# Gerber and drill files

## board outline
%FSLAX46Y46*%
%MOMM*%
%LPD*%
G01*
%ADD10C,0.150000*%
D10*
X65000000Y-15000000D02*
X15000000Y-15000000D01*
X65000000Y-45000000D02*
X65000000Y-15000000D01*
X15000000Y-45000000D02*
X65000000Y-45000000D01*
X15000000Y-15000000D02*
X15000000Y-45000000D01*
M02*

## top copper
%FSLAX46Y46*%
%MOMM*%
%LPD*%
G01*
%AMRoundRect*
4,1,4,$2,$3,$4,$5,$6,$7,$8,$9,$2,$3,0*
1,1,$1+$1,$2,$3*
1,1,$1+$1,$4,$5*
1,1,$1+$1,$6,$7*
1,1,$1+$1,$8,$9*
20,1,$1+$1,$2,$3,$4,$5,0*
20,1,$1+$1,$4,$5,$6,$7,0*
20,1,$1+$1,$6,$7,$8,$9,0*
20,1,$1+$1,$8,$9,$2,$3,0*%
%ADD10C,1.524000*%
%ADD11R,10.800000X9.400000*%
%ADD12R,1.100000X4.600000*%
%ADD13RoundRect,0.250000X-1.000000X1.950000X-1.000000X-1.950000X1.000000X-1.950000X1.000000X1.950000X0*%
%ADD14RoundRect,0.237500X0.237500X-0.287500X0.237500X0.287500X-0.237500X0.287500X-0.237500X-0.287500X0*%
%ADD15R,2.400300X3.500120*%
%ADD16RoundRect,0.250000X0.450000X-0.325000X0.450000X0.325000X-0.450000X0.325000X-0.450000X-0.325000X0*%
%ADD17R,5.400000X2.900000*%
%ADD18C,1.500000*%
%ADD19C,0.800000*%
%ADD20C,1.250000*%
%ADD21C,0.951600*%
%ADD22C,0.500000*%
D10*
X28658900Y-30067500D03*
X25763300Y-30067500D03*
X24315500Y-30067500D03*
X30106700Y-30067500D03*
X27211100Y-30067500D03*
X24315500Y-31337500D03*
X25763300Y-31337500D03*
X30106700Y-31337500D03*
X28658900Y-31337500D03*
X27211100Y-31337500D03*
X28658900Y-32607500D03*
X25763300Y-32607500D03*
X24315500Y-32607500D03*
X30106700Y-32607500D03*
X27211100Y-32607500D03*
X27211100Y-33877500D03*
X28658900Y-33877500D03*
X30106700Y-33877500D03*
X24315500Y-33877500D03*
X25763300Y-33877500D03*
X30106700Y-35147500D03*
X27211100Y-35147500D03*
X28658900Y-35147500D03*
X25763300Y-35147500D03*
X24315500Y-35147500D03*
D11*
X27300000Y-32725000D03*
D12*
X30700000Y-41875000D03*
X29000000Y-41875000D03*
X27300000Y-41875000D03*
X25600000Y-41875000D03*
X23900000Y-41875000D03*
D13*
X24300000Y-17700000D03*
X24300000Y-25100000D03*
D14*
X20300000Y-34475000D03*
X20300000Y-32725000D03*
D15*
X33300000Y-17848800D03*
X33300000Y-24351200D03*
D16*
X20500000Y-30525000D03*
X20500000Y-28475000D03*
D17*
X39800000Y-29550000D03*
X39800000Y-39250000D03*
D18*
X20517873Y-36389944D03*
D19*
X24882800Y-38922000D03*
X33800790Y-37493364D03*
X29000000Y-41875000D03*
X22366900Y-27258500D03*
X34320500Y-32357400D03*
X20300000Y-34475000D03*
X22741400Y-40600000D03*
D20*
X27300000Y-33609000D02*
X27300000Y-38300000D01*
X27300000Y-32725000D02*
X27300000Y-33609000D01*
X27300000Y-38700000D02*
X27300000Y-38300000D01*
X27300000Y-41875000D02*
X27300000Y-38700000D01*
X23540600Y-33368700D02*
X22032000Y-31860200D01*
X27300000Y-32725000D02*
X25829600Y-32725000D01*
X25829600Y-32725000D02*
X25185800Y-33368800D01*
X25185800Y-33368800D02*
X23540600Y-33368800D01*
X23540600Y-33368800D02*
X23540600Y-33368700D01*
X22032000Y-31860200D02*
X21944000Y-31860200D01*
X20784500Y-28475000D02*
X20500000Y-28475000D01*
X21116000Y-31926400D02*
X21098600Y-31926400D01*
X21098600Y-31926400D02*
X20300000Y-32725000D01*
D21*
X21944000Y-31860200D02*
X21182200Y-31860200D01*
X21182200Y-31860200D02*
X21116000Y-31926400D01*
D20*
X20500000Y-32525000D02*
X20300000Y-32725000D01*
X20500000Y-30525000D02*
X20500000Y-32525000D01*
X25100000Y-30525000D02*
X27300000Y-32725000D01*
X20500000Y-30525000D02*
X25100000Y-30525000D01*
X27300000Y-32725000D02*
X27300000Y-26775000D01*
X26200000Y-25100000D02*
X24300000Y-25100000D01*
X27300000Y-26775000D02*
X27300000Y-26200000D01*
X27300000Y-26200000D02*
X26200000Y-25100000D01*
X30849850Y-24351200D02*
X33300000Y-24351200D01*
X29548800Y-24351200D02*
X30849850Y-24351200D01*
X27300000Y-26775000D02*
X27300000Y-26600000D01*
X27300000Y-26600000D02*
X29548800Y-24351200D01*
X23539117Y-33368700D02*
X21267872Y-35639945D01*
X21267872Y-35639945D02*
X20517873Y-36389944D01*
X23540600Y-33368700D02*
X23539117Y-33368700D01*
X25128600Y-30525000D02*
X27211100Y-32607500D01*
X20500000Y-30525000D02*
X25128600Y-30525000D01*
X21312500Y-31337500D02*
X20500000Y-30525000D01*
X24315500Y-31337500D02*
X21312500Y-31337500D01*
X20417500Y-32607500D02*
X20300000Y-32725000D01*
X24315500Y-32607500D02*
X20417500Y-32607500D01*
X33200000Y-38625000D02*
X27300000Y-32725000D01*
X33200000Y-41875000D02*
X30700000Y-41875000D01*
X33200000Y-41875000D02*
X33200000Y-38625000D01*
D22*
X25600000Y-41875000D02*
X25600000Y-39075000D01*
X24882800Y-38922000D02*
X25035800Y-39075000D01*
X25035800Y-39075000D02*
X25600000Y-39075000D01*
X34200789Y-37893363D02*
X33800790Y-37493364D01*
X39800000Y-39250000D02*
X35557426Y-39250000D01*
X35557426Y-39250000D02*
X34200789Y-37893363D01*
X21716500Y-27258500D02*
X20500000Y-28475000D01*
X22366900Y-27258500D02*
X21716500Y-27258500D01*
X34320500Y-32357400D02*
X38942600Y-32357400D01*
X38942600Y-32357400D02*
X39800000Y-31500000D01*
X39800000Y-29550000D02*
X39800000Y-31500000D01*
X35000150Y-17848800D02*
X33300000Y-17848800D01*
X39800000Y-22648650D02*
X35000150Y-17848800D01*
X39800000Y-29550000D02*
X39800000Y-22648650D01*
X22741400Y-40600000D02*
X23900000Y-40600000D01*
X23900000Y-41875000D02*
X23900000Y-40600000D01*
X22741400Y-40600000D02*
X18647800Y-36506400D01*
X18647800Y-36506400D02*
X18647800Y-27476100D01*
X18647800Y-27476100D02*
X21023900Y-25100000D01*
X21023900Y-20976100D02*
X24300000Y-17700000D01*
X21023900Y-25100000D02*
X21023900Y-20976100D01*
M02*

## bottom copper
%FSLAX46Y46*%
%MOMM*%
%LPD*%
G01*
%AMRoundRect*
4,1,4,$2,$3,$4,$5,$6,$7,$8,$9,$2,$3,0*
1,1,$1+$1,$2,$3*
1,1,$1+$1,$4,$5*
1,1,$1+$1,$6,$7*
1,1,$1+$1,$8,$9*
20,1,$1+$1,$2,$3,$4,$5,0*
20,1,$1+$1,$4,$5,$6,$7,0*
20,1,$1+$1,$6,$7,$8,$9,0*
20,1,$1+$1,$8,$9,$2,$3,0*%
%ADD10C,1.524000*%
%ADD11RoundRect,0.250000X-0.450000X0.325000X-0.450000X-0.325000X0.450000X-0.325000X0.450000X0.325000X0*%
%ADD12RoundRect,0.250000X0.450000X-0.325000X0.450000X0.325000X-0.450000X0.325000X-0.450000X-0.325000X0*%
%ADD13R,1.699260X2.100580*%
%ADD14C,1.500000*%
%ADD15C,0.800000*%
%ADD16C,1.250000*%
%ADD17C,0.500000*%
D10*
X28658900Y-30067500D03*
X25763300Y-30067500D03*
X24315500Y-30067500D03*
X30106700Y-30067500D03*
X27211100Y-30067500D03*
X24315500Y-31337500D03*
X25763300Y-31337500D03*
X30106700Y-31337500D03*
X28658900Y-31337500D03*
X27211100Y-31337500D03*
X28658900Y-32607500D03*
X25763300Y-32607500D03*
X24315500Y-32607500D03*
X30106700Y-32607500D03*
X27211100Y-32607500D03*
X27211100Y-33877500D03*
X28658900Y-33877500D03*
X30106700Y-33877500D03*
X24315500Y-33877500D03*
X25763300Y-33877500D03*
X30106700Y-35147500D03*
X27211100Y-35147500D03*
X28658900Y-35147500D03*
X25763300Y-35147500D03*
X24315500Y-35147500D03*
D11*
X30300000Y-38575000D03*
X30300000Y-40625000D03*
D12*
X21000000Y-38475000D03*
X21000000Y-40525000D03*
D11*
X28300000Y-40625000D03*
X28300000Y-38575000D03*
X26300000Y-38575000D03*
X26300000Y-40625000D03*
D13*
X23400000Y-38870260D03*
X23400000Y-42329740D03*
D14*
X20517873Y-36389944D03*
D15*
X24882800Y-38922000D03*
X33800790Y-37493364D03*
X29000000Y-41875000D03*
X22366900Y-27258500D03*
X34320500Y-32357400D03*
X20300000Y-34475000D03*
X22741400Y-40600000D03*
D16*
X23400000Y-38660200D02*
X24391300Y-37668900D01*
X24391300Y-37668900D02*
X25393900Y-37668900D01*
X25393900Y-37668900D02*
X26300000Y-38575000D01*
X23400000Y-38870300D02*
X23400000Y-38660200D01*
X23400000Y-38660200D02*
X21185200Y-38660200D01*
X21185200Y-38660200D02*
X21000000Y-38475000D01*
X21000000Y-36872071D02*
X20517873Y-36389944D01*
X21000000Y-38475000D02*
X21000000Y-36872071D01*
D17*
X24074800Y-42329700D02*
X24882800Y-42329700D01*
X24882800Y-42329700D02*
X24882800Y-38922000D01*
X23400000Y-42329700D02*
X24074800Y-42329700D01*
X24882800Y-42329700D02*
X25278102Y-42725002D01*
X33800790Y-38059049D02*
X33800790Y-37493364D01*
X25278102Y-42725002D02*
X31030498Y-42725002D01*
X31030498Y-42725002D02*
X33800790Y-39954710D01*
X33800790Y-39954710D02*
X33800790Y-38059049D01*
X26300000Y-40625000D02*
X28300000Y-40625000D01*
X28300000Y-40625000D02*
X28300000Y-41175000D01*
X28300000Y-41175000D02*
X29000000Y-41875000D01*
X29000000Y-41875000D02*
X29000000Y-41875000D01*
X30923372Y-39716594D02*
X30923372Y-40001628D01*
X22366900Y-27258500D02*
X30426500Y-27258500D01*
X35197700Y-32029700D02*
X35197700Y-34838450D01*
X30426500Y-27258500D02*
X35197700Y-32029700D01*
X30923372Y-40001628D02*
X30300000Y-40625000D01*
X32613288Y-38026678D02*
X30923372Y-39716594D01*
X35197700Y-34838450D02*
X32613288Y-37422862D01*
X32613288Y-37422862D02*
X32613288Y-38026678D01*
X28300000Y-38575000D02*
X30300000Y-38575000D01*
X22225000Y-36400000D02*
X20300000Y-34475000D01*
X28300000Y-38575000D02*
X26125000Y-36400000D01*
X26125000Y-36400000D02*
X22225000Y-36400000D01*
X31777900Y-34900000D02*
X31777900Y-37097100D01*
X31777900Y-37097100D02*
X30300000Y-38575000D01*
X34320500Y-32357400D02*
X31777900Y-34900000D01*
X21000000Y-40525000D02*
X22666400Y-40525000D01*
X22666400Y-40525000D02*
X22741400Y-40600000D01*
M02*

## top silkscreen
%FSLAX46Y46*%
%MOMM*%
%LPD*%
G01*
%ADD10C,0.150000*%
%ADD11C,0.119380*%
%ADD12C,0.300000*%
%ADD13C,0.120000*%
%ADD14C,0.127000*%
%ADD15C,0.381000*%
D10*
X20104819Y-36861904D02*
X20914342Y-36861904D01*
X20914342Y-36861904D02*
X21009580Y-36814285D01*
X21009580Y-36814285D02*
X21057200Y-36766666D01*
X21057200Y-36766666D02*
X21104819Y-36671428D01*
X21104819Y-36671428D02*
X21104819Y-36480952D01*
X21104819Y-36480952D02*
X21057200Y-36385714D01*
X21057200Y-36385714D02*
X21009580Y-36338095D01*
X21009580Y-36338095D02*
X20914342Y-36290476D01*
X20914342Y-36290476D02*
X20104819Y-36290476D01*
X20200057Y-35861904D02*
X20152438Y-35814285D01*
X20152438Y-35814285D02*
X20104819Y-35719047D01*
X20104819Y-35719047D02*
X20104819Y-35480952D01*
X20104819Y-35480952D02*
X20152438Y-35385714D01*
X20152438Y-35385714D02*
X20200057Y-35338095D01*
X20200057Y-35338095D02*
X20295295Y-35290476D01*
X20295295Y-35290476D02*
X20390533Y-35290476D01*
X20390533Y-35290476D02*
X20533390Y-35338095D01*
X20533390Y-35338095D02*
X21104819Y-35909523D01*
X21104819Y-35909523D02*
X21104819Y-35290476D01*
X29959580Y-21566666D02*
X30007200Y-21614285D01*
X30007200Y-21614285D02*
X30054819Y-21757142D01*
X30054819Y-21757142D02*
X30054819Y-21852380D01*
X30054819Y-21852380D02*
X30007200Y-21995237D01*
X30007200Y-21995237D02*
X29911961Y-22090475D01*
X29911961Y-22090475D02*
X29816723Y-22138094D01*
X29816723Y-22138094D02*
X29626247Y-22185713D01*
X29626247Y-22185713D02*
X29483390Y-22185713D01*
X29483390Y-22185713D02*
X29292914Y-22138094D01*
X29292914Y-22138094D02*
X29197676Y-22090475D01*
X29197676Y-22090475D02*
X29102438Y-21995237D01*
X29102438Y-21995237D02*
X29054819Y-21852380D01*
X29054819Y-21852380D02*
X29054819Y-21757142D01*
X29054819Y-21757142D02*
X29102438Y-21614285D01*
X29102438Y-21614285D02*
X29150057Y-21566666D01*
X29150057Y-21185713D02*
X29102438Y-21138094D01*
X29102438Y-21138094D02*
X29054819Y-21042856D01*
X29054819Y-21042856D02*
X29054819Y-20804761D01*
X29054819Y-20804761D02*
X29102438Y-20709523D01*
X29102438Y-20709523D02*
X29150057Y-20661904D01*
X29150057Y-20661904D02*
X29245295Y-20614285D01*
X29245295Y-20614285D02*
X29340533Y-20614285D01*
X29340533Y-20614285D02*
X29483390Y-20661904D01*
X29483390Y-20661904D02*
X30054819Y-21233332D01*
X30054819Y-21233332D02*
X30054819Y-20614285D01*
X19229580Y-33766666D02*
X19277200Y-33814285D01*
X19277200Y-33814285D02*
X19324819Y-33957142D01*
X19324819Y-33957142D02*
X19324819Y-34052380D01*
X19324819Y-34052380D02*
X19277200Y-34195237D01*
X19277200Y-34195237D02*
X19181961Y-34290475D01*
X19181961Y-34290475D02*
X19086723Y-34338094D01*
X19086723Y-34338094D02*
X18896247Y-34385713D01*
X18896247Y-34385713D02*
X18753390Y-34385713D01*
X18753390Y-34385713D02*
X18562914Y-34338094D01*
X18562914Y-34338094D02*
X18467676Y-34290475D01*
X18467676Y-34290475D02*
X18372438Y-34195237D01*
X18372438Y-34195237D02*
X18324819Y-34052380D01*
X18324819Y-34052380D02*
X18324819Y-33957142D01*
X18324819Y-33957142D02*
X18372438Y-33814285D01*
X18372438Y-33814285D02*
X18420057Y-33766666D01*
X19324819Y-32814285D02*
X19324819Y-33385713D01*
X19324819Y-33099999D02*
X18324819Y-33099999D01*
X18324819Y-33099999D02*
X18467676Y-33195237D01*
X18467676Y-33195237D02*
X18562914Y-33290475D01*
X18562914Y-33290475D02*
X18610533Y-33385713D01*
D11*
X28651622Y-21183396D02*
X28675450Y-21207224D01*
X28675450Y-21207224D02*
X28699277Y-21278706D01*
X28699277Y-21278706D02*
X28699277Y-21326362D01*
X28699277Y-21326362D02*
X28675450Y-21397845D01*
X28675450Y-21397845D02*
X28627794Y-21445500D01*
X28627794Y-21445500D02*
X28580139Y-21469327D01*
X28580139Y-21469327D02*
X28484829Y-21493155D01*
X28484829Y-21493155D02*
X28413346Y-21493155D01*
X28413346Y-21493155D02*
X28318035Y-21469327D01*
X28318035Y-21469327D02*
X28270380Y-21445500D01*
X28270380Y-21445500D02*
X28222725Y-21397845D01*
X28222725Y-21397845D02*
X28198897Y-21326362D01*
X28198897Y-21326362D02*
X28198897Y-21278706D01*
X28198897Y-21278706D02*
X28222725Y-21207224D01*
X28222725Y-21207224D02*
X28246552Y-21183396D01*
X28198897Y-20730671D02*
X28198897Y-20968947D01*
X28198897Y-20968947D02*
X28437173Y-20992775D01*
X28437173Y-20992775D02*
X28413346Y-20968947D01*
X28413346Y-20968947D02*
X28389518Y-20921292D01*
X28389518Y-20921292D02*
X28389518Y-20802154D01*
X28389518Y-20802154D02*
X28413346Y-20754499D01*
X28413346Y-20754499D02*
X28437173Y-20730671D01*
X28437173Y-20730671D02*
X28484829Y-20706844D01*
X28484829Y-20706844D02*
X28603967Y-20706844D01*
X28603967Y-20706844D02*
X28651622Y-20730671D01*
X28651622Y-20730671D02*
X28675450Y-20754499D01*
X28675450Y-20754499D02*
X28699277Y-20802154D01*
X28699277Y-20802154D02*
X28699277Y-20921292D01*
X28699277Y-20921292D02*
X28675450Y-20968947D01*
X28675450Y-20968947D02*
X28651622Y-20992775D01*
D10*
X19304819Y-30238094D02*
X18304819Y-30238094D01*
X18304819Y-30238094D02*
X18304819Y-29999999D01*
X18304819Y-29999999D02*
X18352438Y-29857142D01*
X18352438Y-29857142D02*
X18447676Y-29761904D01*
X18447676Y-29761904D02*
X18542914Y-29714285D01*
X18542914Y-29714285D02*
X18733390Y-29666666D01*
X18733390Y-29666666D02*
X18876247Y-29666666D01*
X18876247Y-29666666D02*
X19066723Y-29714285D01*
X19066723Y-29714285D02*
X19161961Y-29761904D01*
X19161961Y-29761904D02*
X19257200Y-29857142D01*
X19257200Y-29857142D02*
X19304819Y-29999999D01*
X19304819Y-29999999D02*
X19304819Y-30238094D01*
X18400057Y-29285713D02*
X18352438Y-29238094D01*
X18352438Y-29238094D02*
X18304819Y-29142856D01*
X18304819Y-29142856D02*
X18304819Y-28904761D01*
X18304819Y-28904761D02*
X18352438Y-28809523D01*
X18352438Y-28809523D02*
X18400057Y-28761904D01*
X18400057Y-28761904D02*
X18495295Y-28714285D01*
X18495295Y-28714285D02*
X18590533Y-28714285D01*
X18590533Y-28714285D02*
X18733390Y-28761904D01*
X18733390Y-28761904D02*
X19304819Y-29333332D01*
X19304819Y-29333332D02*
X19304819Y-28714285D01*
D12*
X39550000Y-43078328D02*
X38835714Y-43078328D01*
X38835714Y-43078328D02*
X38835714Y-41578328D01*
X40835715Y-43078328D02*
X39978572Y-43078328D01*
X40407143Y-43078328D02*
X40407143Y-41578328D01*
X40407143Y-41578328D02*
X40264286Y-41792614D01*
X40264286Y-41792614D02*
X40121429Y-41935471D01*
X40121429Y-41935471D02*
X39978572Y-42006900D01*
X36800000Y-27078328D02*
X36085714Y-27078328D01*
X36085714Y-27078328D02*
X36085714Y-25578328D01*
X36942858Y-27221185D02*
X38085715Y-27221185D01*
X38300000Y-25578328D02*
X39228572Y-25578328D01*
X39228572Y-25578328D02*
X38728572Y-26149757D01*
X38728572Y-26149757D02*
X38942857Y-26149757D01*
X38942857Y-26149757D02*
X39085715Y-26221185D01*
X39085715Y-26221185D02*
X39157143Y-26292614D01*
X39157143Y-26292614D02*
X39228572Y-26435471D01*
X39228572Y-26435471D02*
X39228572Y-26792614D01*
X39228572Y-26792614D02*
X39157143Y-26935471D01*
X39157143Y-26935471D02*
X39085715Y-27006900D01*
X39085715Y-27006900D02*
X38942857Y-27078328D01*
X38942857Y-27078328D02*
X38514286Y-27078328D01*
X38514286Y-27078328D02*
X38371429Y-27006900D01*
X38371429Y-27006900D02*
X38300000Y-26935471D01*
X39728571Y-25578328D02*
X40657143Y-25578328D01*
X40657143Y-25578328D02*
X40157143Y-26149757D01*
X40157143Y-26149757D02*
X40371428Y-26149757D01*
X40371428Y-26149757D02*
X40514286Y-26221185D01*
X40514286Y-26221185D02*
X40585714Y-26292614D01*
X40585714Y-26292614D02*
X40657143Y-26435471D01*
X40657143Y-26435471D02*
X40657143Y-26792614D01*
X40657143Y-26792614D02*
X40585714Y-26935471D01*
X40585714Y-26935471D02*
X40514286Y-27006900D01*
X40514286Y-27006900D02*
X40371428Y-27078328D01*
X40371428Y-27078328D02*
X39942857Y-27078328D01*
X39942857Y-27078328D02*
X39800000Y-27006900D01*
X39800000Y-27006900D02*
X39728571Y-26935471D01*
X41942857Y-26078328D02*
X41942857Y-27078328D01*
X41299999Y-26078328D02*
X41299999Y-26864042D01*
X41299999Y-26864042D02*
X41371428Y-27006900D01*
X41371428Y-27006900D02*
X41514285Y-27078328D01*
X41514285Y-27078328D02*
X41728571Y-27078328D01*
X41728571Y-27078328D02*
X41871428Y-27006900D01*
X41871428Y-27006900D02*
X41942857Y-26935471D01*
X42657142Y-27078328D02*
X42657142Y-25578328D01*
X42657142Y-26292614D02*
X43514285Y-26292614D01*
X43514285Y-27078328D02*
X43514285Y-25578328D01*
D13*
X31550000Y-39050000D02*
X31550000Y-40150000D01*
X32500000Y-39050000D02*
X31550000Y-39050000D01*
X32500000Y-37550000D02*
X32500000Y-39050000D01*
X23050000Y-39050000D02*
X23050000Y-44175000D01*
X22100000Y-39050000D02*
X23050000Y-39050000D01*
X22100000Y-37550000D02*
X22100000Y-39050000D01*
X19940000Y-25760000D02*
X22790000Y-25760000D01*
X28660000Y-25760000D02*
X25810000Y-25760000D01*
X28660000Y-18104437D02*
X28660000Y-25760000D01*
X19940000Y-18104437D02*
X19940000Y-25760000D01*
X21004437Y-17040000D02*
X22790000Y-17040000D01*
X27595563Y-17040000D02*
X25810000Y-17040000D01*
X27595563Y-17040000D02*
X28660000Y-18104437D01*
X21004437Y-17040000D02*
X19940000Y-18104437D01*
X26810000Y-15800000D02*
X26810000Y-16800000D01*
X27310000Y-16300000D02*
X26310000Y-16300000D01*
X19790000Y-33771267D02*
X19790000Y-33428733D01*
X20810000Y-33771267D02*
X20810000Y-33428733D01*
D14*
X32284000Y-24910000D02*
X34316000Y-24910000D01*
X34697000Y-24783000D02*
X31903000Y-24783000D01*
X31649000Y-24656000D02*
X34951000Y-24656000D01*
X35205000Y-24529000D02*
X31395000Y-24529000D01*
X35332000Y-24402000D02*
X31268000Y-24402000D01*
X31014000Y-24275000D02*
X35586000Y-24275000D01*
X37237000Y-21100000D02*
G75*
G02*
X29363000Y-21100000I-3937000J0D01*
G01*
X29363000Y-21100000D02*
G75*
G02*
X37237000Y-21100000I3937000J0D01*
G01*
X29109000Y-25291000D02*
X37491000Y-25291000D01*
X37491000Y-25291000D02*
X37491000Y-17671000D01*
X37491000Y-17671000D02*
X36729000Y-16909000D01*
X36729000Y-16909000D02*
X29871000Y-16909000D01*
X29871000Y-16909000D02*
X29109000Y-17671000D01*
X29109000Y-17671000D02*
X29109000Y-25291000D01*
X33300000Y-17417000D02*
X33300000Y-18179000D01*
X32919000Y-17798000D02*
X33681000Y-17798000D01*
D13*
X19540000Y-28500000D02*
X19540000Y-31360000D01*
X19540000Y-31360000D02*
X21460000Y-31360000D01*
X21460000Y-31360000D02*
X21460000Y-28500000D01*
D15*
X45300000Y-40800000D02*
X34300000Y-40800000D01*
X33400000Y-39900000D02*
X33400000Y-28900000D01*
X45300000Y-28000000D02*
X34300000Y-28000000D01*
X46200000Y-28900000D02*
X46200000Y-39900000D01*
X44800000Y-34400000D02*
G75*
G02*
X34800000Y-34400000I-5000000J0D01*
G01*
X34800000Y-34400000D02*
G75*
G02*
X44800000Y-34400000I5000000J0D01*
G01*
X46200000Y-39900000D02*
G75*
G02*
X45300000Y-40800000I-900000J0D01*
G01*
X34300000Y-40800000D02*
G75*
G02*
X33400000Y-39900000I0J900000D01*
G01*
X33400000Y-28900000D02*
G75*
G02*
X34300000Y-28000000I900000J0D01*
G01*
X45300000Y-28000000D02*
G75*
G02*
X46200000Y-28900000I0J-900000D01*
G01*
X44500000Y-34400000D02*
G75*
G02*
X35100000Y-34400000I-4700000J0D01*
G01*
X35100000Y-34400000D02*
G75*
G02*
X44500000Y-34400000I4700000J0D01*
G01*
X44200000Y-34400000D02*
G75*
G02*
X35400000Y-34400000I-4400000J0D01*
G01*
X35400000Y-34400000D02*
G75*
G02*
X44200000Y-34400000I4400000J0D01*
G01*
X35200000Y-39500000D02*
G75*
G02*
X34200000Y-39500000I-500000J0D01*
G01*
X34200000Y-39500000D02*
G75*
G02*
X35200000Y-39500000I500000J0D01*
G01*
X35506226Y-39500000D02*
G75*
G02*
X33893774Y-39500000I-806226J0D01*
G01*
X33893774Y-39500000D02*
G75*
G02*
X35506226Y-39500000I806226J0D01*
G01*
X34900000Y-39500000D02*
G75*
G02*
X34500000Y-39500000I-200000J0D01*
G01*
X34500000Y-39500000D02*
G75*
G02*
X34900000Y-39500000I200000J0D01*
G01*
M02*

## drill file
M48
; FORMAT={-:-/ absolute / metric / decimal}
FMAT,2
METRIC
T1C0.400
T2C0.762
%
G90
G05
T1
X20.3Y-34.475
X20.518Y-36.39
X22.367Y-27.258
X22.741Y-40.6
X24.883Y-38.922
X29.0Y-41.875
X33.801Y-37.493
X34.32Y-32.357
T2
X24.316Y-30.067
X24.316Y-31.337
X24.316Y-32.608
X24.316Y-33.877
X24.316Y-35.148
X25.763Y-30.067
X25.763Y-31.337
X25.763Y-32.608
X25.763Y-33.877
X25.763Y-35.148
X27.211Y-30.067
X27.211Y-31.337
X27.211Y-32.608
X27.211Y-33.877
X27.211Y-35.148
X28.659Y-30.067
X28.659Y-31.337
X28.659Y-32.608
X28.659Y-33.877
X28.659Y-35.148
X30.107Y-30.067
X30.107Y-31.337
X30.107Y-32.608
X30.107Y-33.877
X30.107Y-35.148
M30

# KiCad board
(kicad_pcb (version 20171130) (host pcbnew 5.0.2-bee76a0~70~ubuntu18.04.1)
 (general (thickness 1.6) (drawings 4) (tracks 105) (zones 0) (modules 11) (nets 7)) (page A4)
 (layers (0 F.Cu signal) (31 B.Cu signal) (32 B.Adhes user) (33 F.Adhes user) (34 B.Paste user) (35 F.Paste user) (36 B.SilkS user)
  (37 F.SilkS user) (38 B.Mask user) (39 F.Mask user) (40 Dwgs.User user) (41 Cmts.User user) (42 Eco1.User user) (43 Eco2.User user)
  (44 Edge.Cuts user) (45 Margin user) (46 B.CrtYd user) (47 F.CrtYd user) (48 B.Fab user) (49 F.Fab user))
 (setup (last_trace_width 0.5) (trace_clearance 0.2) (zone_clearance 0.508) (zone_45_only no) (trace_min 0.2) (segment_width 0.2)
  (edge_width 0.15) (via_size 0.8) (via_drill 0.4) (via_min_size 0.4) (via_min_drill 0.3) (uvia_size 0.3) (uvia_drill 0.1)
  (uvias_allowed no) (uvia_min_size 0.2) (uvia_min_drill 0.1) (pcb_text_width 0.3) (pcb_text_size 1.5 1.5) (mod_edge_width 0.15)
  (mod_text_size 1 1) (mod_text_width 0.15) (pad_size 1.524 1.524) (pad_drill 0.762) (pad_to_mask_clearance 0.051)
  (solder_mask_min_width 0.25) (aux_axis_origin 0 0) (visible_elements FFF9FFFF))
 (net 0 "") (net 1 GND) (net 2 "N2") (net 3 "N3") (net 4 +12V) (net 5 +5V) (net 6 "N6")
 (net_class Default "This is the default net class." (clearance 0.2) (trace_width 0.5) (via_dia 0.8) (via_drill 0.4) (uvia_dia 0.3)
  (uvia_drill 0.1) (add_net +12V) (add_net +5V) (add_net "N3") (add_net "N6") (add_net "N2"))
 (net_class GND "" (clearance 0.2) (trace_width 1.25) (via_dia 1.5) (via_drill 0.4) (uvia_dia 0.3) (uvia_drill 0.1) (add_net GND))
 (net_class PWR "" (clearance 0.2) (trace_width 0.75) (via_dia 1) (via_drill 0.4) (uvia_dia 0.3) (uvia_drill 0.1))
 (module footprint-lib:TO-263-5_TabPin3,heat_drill (layer F.Cu) (at 27.3 36.1 90)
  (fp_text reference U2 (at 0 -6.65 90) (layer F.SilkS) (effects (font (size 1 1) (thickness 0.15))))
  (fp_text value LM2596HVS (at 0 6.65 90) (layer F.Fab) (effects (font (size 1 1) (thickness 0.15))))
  (fp_line (start -2.95 4.25) (end -4.05 4.25) (layer F.SilkS) (width 0.12))
  (fp_line (start -2.95 5.2) (end -2.95 4.25) (layer F.SilkS) (width 0.12))
  (fp_line (start -1.45 5.2) (end -2.95 5.2) (layer F.SilkS) (width 0.12))
  (fp_line (start -2.95 -4.25) (end -8.075 -4.25) (layer F.SilkS) (width 0.12))
  (fp_line (start -2.95 -5.2) (end -2.95 -4.25) (layer F.SilkS) (width 0.12))
  (fp_line (start -1.45 -5.2) (end -2.95 -5.2) (layer F.SilkS) (width 0.12))
  (pad 3 thru_hole circle (at 6.0325 1.3589 90) (size 1.524 1.524) (drill 0.762) (layers *.Cu *.Mask) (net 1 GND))
  (pad 3 thru_hole circle (at 6.0325 -1.5367 90) (size 1.524 1.524) (drill 0.762) (layers *.Cu *.Mask) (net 1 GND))
  (pad 3 thru_hole circle (at 6.0325 -2.9845 90) (size 1.524 1.524) (drill 0.762) (layers *.Cu *.Mask) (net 1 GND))
  (pad 3 thru_hole circle (at 6.0325 2.8067 90) (size 1.524 1.524) (drill 0.762) (layers *.Cu *.Mask) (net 1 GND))
  (pad 3 thru_hole circle (at 6.0325 -0.0889 90) (size 1.524 1.524) (drill 0.762) (layers *.Cu *.Mask) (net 1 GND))
  (pad 3 thru_hole circle (at 4.7625 -2.9845 90) (size 1.524 1.524) (drill 0.762) (layers *.Cu *.Mask) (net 1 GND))
  (pad 3 thru_hole circle (at 4.7625 -1.5367 90) (size 1.524 1.524) (drill 0.762) (layers *.Cu *.Mask) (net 1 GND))
  (pad 3 thru_hole circle (at 4.7625 2.8067 90) (size 1.524 1.524) (drill 0.762) (layers *.Cu *.Mask) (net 1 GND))
  (pad 3 thru_hole circle (at 4.7625 1.3589 90) (size 1.524 1.524) (drill 0.762) (layers *.Cu *.Mask) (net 1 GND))
  (pad 3 thru_hole circle (at 4.7625 -0.0889 90) (size 1.524 1.524) (drill 0.762) (layers *.Cu *.Mask) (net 1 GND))
  (pad 3 thru_hole circle (at 3.4925 1.3589 90) (size 1.524 1.524) (drill 0.762) (layers *.Cu *.Mask) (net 1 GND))
  (pad 3 thru_hole circle (at 3.4925 -1.5367 90) (size 1.524 1.524) (drill 0.762) (layers *.Cu *.Mask) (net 1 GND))
  (pad 3 thru_hole circle (at 3.4925 -2.9845 90) (size 1.524 1.524) (drill 0.762) (layers *.Cu *.Mask) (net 1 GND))
  (pad 3 thru_hole circle (at 3.4925 2.8067 90) (size 1.524 1.524) (drill 0.762) (layers *.Cu *.Mask) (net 1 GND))
  (pad 3 thru_hole circle (at 3.4925 -0.0889 90) (size 1.524 1.524) (drill 0.762) (layers *.Cu *.Mask) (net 1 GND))
  (pad 3 thru_hole circle (at 2.2225 -0.0889 90) (size 1.524 1.524) (drill 0.762) (layers *.Cu *.Mask) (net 1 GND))
  (pad 3 thru_hole circle (at 2.2225 1.3589 90) (size 1.524 1.524) (drill 0.762) (layers *.Cu *.Mask) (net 1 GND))
  (pad 3 thru_hole circle (at 2.2225 2.8067 90) (size 1.524 1.524) (drill 0.762) (layers *.Cu *.Mask) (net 1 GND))
  (pad 3 thru_hole circle (at 2.2225 -2.9845 90) (size 1.524 1.524) (drill 0.762) (layers *.Cu *.Mask) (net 1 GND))
  (pad 3 thru_hole circle (at 2.2225 -1.5367 90) (size 1.524 1.524) (drill 0.762) (layers *.Cu *.Mask) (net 1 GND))
  (pad 3 thru_hole circle (at 0.9525 2.8067 90) (size 1.524 1.524) (drill 0.762) (layers *.Cu *.Mask) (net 1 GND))
  (pad 3 thru_hole circle (at 0.9525 -0.0889 90) (size 1.524 1.524) (drill 0.762) (layers *.Cu *.Mask) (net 1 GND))
  (pad 3 thru_hole circle (at 0.9525 1.3589 90) (size 1.524 1.524) (drill 0.762) (layers *.Cu *.Mask) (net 1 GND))
  (pad 3 thru_hole circle (at 0.9525 -1.5367 90) (size 1.524 1.524) (drill 0.762) (layers *.Cu *.Mask) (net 1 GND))
  (pad 3 thru_hole circle (at 0.9525 -2.9845 90) (size 1.524 1.524) (drill 0.762) (layers *.Cu *.Mask) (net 1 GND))
  (pad "" smd rect (at 0.95 2.775 90) (size 4.55 5.25) (layers F.Paste))
  (pad "" smd rect (at 5.8 -2.775 90) (size 4.55 5.25) (layers F.Paste))
  (pad "" smd rect (at 0.95 -2.775 90) (size 4.55 5.25) (layers F.Paste))
  (pad "" smd rect (at 5.8 2.775 90) (size 4.55 5.25) (layers F.Paste))
  (pad 3 smd rect (at 3.375 0 90) (size 9.4 10.8) (layers F.Cu F.Mask) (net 1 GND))
  (pad 5 smd rect (at -5.775 3.4 90) (size 4.6 1.1) (layers F.Cu F.Paste F.Mask) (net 1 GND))
  (pad 4 smd rect (at -5.775 1.7 90) (size 4.6 1.1) (layers F.Cu F.Paste F.Mask) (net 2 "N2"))
  (pad 3 smd rect (at -5.775 0 90) (size 4.6 1.1) (layers F.Cu F.Paste F.Mask) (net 1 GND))
  (pad 2 smd rect (at -5.775 -1.7 90) (size 4.6 1.1) (layers F.Cu F.Paste F.Mask) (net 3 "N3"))
  (pad 1 smd rect (at -5.775 -3.4 90) (size 4.6 1.1) (layers F.Cu F.Paste F.Mask) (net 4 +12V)))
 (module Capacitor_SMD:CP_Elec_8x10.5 (layer F.Cu) (at 24.3 21.4 270)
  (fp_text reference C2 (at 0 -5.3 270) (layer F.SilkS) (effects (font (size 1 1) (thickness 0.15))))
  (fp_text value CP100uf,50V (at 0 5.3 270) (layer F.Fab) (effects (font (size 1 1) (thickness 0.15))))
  (fp_line (start 4.36 4.36) (end 4.36 1.51) (layer F.SilkS) (width 0.12))
  (fp_line (start 4.36 -4.36) (end 4.36 -1.51) (layer F.SilkS) (width 0.12))
  (fp_line (start -3.295563 -4.36) (end 4.36 -4.36) (layer F.SilkS) (width 0.12))
  (fp_line (start -3.295563 4.36) (end 4.36 4.36) (layer F.SilkS) (width 0.12))
  (fp_line (start -4.36 3.295563) (end -4.36 1.51) (layer F.SilkS) (width 0.12))
  (fp_line (start -4.36 -3.295563) (end -4.36 -1.51) (layer F.SilkS) (width 0.12))
  (fp_line (start -4.36 -3.295563) (end -3.295563 -4.36) (layer F.SilkS) (width 0.12))
  (fp_line (start -4.36 3.295563) (end -3.295563 4.36) (layer F.SilkS) (width 0.12))
  (fp_line (start -5.6 -2.51) (end -4.6 -2.51) (layer F.SilkS) (width 0.12))
  (fp_line (start -5.1 -3.01) (end -5.1 -2.01) (layer F.SilkS) (width 0.12))
  (pad 1 smd roundrect (at -3.7 0 270) (size 4.4 2.5) (layers F.Cu F.Paste F.Mask) (roundrect_rratio 0.1) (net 4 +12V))
  (pad 2 smd roundrect (at 3.7 0 270) (size 4.4 2.5) (layers F.Cu F.Paste F.Mask) (roundrect_rratio 0.1) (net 1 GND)))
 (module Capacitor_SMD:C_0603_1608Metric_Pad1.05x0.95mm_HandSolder (layer F.Cu) (at 20.3 33.6 90)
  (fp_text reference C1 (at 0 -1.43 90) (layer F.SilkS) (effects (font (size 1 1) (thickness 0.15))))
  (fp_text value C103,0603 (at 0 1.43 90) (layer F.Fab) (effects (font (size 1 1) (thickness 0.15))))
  (fp_line (start -0.171267 -0.51) (end 0.171267 -0.51) (layer F.SilkS) (width 0.12))
  (fp_line (start -0.171267 0.51) (end 0.171267 0.51) (layer F.SilkS) (width 0.12))
  (pad 1 smd roundrect (at -0.875 0 90) (size 1.05 0.95) (layers F.Cu F.Paste F.Mask) (roundrect_rratio 0.25) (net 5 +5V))
  (pad 2 smd roundrect (at 0.875 0 90) (size 1.05 0.95) (layers F.Cu F.Paste F.Mask) (roundrect_rratio 0.25) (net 1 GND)))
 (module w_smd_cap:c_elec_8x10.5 (layer F.Cu) (at 33.3 21.1 90)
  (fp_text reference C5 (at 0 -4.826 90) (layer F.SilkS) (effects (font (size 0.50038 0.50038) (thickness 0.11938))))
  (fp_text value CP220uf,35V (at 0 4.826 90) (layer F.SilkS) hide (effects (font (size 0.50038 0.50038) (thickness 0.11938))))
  (fp_line (start -3.81 -1.016) (end -3.81 1.016) (layer F.SilkS) (width 0.127))
  (fp_line (start -3.683 1.397) (end -3.683 -1.397) (layer F.SilkS) (width 0.127))
  (fp_line (start -3.556 -1.651) (end -3.556 1.651) (layer F.SilkS) (width 0.127))
  (fp_line (start -3.429 1.905) (end -3.429 -1.905) (layer F.SilkS) (width 0.127))
  (fp_line (start -3.302 2.032) (end -3.302 -2.032) (layer F.SilkS) (width 0.127))
  (fp_line (start -3.175 -2.286) (end -3.175 2.286) (layer F.SilkS) (width 0.127))
  (fp_circle (center 0 0) (end 3.937 0) (layer F.SilkS) (width 0.127))
  (fp_line (start -4.191 -4.191) (end -4.191 4.191) (layer F.SilkS) (width 0.127))
  (fp_line (start -4.191 4.191) (end 3.429 4.191) (layer F.SilkS) (width 0.127))
  (fp_line (start 3.429 4.191) (end 4.191 3.429) (layer F.SilkS) (width 0.127))
  (fp_line (start 4.191 3.429) (end 4.191 -3.429) (layer F.SilkS) (width 0.127))
  (fp_line (start 4.191 -3.429) (end 3.429 -4.191) (layer F.SilkS) (width 0.127))
  (fp_line (start 3.429 -4.191) (end -4.191 -4.191) (layer F.SilkS) (width 0.127))
  (fp_line (start 3.683 0) (end 2.921 0) (layer F.SilkS) (width 0.127))
  (fp_line (start 3.302 -0.381) (end 3.302 0.381) (layer F.SilkS) (width 0.127))
  (pad 1 smd rect (at 3.2512 0 90) (size 3.50012 2.4003) (layers F.Cu F.Paste F.Mask) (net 5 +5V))
  (pad 2 smd rect (at -3.2512 0 90) (size 3.50012 2.4003) (layers F.Cu F.Paste F.Mask) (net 1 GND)))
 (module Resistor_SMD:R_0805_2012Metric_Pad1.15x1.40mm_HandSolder (layer B.Cu) (at 30.3 39.6 270)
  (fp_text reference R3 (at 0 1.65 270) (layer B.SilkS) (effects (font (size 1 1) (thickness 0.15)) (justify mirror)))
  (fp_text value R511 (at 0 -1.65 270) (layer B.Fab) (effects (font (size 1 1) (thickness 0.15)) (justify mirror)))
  (pad 1 smd roundrect (at -1.025 0 270) (size 1.15 1.4) (layers B.Cu B.Paste B.Mask) (roundrect_rratio 0.217391) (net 5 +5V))
  (pad 2 smd roundrect (at 1.025 0 270) (size 1.15 1.4) (layers B.Cu B.Paste B.Mask) (roundrect_rratio 0.217391) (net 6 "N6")))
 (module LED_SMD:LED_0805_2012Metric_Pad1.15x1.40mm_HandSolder (layer F.Cu) (at 20.5 29.5 90)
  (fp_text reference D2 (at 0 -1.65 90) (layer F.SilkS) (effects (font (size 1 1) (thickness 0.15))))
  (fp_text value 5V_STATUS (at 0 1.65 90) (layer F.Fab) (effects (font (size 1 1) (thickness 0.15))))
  (fp_line (start 1 -0.96) (end -1.86 -0.96) (layer F.SilkS) (width 0.12))
  (fp_line (start -1.86 -0.96) (end -1.86 0.96) (layer F.SilkS) (width 0.12))
  (fp_line (start -1.86 0.96) (end 1 0.96) (layer F.SilkS) (width 0.12))
  (pad 1 smd roundrect (at -1.025 0 90) (size 1.15 1.4) (layers F.Cu F.Paste F.Mask) (roundrect_rratio 0.217391) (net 1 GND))
  (pad 2 smd roundrect (at 1.025 0 90) (size 1.15 1.4) (layers F.Cu F.Paste F.Mask) (roundrect_rratio 0.217391) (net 6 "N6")))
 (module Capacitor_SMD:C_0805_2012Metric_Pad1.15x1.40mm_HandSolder (layer B.Cu) (at 21 39.5 90)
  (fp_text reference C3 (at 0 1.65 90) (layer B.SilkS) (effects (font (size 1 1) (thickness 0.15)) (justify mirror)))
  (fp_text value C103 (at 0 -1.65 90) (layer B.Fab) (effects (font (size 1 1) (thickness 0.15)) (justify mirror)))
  (pad 2 smd roundrect (at 1.025 0 90) (size 1.15 1.4) (layers B.Cu B.Paste B.Mask) (roundrect_rratio 0.217391) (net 1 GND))
  (pad 1 smd roundrect (at -1.025 0 90) (size 1.15 1.4) (layers B.Cu B.Paste B.Mask) (roundrect_rratio 0.217391) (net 4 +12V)))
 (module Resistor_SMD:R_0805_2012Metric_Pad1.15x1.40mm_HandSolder (layer B.Cu) (at 28.3 39.6 270)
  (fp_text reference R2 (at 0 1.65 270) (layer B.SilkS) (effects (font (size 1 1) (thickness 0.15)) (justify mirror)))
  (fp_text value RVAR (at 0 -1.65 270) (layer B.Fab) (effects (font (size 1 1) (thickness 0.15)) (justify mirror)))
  (pad 2 smd roundrect (at 1.025 0 270) (size 1.15 1.4) (layers B.Cu B.Paste B.Mask) (roundrect_rratio 0.217391) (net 2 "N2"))
  (pad 1 smd roundrect (at -1.025 0 270) (size 1.15 1.4) (layers B.Cu B.Paste B.Mask) (roundrect_rratio 0.217391) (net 5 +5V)))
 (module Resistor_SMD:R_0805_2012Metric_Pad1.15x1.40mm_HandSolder (layer B.Cu) (at 26.3 39.6 270)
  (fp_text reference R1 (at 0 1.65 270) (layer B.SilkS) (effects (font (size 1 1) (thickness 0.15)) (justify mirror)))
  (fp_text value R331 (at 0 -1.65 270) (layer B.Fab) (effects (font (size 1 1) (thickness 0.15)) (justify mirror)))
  (pad 1 smd roundrect (at -1.025 0 270) (size 1.15 1.4) (layers B.Cu B.Paste B.Mask) (roundrect_rratio 0.217391) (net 1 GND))
  (pad 2 smd roundrect (at 1.025 0 270) (size 1.15 1.4) (layers B.Cu B.Paste B.Mask) (roundrect_rratio 0.217391) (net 2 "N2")))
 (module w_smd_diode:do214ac (layer B.Cu) (at 23.4 40.6 90)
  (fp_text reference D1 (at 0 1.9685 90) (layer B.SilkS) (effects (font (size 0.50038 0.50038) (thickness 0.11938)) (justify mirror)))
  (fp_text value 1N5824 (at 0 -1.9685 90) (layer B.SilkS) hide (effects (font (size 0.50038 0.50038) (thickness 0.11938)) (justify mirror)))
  (pad 2 smd rect (at 1.72974 0 90) (size 2.10058 1.69926) (layers B.Cu B.Paste B.Mask) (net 1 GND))
  (pad 1 smd rect (at -1.72974 0 90) (size 2.10058 1.69926) (layers B.Cu B.Paste B.Mask) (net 3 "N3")))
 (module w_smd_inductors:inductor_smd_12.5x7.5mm (layer F.Cu) (at 39.8 34.4 180)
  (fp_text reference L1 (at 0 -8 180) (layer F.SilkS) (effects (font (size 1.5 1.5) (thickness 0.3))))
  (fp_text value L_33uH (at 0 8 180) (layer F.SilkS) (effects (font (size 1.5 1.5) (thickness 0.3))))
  (fp_line (start -5.5 -6.4) (end 5.5 -6.4) (layer F.SilkS) (width 0.381))
  (fp_line (start 6.4 -5.5) (end 6.4 5.5) (layer F.SilkS) (width 0.381))
  (fp_line (start -5.5 6.4) (end 5.5 6.4) (layer F.SilkS) (width 0.381))
  (fp_line (start -6.4 5.5) (end -6.4 -5.5) (layer F.SilkS) (width 0.381))
  (fp_circle (center 0 0) (end 5 0) (layer F.SilkS) (width 0.381))
  (fp_arc (start -5.5 -5.5) (end -6.4 -5.5) (angle 90) (layer F.SilkS) (width 0.381))
  (fp_arc (start 5.5 -5.5) (end 5.5 -6.4) (angle 90) (layer F.SilkS) (width 0.381))
  (fp_arc (start 5.5 5.5) (end 6.4 5.5) (angle 90) (layer F.SilkS) (width 0.381))
  (fp_arc (start -5.5 5.5) (end -5.5 6.4) (angle 90) (layer F.SilkS) (width 0.381))
  (fp_circle (center 0 0) (end 4.7 0) (layer F.SilkS) (width 0.381))
  (fp_circle (center 0 0) (end 4.4 0) (layer F.SilkS) (width 0.381))
  (fp_circle (center 5.1 -5.1) (end 5.6 -5.1) (layer F.SilkS) (width 0.381))
  (fp_circle (center 5.1 -5.1) (end 5.9 -5) (layer F.SilkS) (width 0.381))
  (fp_circle (center 5.1 -5.1) (end 5.3 -5.1) (layer F.SilkS) (width 0.381))
  (pad 2 smd rect (at 0 4.85 180) (size 5.4 2.9) (layers F.Cu F.Paste F.Mask) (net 5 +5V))
  (pad 1 smd rect (at 0 -4.85 180) (size 5.4 2.9) (layers F.Cu F.Paste F.Mask) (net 3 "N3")))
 (gr_line (start 65 15) (end 15 15) (layer Edge.Cuts) (width 0.15))
 (gr_line (start 65 45) (end 65 15) (layer Edge.Cuts) (width 0.15))
 (gr_line (start 15 45) (end 65 45) (layer Edge.Cuts) (width 0.15))
 (gr_line (start 15 15) (end 15 45) (layer Edge.Cuts) (width 0.15))
 (segment (start 23.4 38.6602) (end 24.3913 37.6689) (width 1.25) (layer B.Cu) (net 1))
 (segment (start 24.3913 37.6689) (end 25.3939 37.6689) (width 1.25) (layer B.Cu) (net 1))
 (segment (start 25.3939 37.6689) (end 26.3 38.575) (width 1.25) (layer B.Cu) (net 1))
 (segment (start 23.4 38.8703) (end 23.4 38.6602) (width 1.25) (layer B.Cu) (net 1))
 (segment (start 23.4 38.6602) (end 21.1852 38.6602) (width 1.25) (layer B.Cu) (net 1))
 (segment (start 21.1852 38.6602) (end 21 38.475) (width 1.25) (layer B.Cu) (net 1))
 (segment (start 27.3 33.609) (end 27.3 38.3) (width 1.25) (layer F.Cu) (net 1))
 (segment (start 27.3 32.725) (end 27.3 33.609) (width 1.25) (layer F.Cu) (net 1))
 (segment (start 27.3 38.7) (end 27.3 38.3) (width 1.25) (layer F.Cu) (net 1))
 (segment (start 27.3 41.875) (end 27.3 38.7) (width 1.25) (layer F.Cu) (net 1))
 (segment (start 23.5406 33.3687) (end 22.032 31.8602) (width 1.25) (layer F.Cu) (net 1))
 (segment (start 27.3 32.725) (end 25.8296 32.725) (width 1.25) (layer F.Cu) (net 1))
 (segment (start 25.8296 32.725) (end 25.1858 33.3688) (width 1.25) (layer F.Cu) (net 1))
 (segment (start 25.1858 33.3688) (end 23.5406 33.3688) (width 1.25) (layer F.Cu) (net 1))
 (segment (start 23.5406 33.3688) (end 23.5406 33.3687) (width 1.25) (layer F.Cu) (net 1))
 (segment (start 22.032 31.8602) (end 21.944 31.8602) (width 1.25) (layer F.Cu) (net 1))
 (segment (start 20.7845 28.475) (end 20.5 28.475) (width 1.25) (layer F.Cu) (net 6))
 (segment (start 21.116 31.9264) (end 21.0986 31.9264) (width 1.25) (layer F.Cu) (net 1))
 (segment (start 21.0986 31.9264) (end 20.3 32.725) (width 1.25) (layer F.Cu) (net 1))
 (segment (start 21.944 31.8602) (end 21.1822 31.8602) (width 0.9516) (layer F.Cu) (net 1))
 (segment (start 21.1822 31.8602) (end 21.116 31.9264) (width 0.9516) (layer F.Cu) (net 1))
 (segment (start 20.5 32.525) (end 20.3 32.725) (width 1.25) (layer F.Cu) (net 1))
 (segment (start 20.5 30.525) (end 20.5 32.525) (width 1.25) (layer F.Cu) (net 1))
 (segment (start 25.1 30.525) (end 27.3 32.725) (width 1.25) (layer F.Cu) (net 1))
 (segment (start 20.5 30.525) (end 25.1 30.525) (width 1.25) (layer F.Cu) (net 1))
 (segment (start 27.3 32.725) (end 27.3 26.775) (width 1.25) (layer F.Cu) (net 1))
 (segment (start 26.2 25.1) (end 24.3 25.1) (width 1.25) (layer F.Cu) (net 1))
 (segment (start 27.3 26.775) (end 27.3 26.2) (width 1.25) (layer F.Cu) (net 1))
 (segment (start 27.3 26.2) (end 26.2 25.1) (width 1.25) (layer F.Cu) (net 1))
 (segment (start 30.84985 24.3512) (end 33.3 24.3512) (width 1.25) (layer F.Cu) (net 1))
 (segment (start 29.5488 24.3512) (end 30.84985 24.3512) (width 1.25) (layer F.Cu) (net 1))
 (segment (start 27.3 26.775) (end 27.3 26.6) (width 1.25) (layer F.Cu) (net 1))
 (segment (start 27.3 26.6) (end 29.5488 24.3512) (width 1.25) (layer F.Cu) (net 1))
 (segment (start 23.539117 33.3687) (end 21.267872 35.639945) (width 1.25) (layer F.Cu) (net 1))
 (segment (start 21.267872 35.639945) (end 20.517873 36.389944) (width 1.25) (layer F.Cu) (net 1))
 (segment (start 23.5406 33.3687) (end 23.539117 33.3687) (width 1.25) (layer F.Cu) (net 1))
 (segment (start 21 36.872071) (end 20.517873 36.389944) (width 1.25) (layer B.Cu) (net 1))
 (via (at 20.517873 36.389944) (size 1.5) (drill 0.4) (layers F.Cu B.Cu) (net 1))
 (segment (start 21 38.475) (end 21 36.872071) (width 1.25) (layer B.Cu) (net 1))
 (segment (start 25.1286 30.525) (end 27.2111 32.6075) (width 1.25) (layer F.Cu) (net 1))
 (segment (start 20.5 30.525) (end 25.1286 30.525) (width 1.25) (layer F.Cu) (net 1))
 (segment (start 21.3125 31.3375) (end 20.5 30.525) (width 1.25) (layer F.Cu) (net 1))
 (segment (start 24.3155 31.3375) (end 21.3125 31.3375) (width 1.25) (layer F.Cu) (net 1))
 (segment (start 20.4175 32.6075) (end 20.3 32.725) (width 1.25) (layer F.Cu) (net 1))
 (segment (start 24.3155 32.6075) (end 20.4175 32.6075) (width 1.25) (layer F.Cu) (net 1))
 (segment (start 33.2 38.625) (end 27.3 32.725) (width 1.25) (layer F.Cu) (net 1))
 (segment (start 33.2 41.875) (end 30.7 41.875) (width 1.25) (layer F.Cu) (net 1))
 (segment (start 33.2 41.875) (end 33.2 38.625) (width 1.25) (layer F.Cu) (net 1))
 (segment (start 24.0748 42.3297) (end 24.8828 42.3297) (width 0.5) (layer B.Cu) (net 3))
 (segment (start 24.8828 42.3297) (end 24.8828 38.922) (width 0.5) (layer B.Cu) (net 3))
 (segment (start 25.6 41.875) (end 25.6 39.075) (width 0.5) (layer F.Cu) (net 3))
 (segment (start 24.8828 38.922) (end 25.0358 39.075) (width 0.5) (layer F.Cu) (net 3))
 (segment (start 25.0358 39.075) (end 25.6 39.075) (width 0.5) (layer F.Cu) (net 3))
 (segment (start 23.4 42.3297) (end 24.0748 42.3297) (width 0.5) (layer B.Cu) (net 3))
 (via (at 24.8828 38.922) (size 0.8) (layers F.Cu B.Cu) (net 3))
 (segment (start 34.200789 37.893363) (end 33.80079 37.493364) (width 0.5) (layer F.Cu) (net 3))
 (segment (start 39.8 39.25) (end 35.557426 39.25) (width 0.5) (layer F.Cu) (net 3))
 (via (at 33.80079 37.493364) (size 0.8) (drill 0.4) (layers F.Cu B.Cu) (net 3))
 (segment (start 35.557426 39.25) (end 34.200789 37.893363) (width 0.5) (layer F.Cu) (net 3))
 (segment (start 24.8828 42.3297) (end 25.278102 42.725002) (width 0.5) (layer B.Cu) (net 3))
 (segment (start 33.80079 38.059049) (end 33.80079 37.493364) (width 0.5) (layer B.Cu) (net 3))
 (segment (start 25.278102 42.725002) (end 31.030498 42.725002) (width 0.5) (layer B.Cu) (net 3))
 (segment (start 31.030498 42.725002) (end 33.80079 39.95471) (width 0.5) (layer B.Cu) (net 3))
 (segment (start 33.80079 39.95471) (end 33.80079 38.059049) (width 0.5) (layer B.Cu) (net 3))
 (segment (start 26.3 40.625) (end 28.3 40.625) (width 0.5) (layer B.Cu) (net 2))
 (segment (start 28.3 40.625) (end 28.3 41.175) (width 0.5) (layer B.Cu) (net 2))
 (segment (start 28.3 41.175) (end 29 41.875) (width 0.5) (layer B.Cu) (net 2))
 (segment (start 29 41.875) (end 29 41.875) (width 0.5) (layer B.Cu) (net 2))
 (via (at 29 41.875) (size 0.8) (drill 0.4) (layers F.Cu B.Cu) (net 2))
 (via (at 22.3669 27.2585) (size 0.8) (layers F.Cu B.Cu) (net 6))
 (segment (start 21.7165 27.2585) (end 20.5 28.475) (width 0.5) (layer F.Cu) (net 6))
 (segment (start 22.3669 27.2585) (end 21.7165 27.2585) (width 0.5) (layer F.Cu) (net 6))
 (segment (start 30.923372 39.716594) (end 30.923372 40.001628) (width 0.5) (layer B.Cu) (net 6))
 (segment (start 22.3669 27.2585) (end 30.4265 27.2585) (width 0.5) (layer B.Cu) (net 6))
 (segment (start 35.1977 32.0297) (end 35.1977 34.83845) (width 0.5) (layer B.Cu) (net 6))
 (segment (start 30.4265 27.2585) (end 35.1977 32.0297) (width 0.5) (layer B.Cu) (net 6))
 (segment (start 30.923372 40.001628) (end 30.3 40.625) (width 0.5) (layer B.Cu) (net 6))
 (segment (start 32.613288 38.026678) (end 30.923372 39.716594) (width 0.5) (layer B.Cu) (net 6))
 (segment (start 35.1977 34.83845) (end 32.613288 37.422862) (width 0.5) (layer B.Cu) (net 6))
 (segment (start 32.613288 37.422862) (end 32.613288 38.026678) (width 0.5) (layer B.Cu) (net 6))
 (segment (start 34.3205 32.3574) (end 38.9426 32.3574) (width 0.5) (layer F.Cu) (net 5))
 (segment (start 38.9426 32.3574) (end 39.8 31.5) (width 0.5) (layer F.Cu) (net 5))
 (segment (start 39.8 29.55) (end 39.8 31.5) (width 0.5) (layer F.Cu) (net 5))
 (segment (start 28.3 38.575) (end 30.3 38.575) (width 0.5) (layer B.Cu) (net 5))
 (via (at 34.3205 32.3574) (size 0.8) (layers F.Cu B.Cu) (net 5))
 (segment (start 35.00015 17.8488) (end 33.3 17.8488) (width 0.5) (layer F.Cu) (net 5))
 (segment (start 39.8 22.64865) (end 35.00015 17.8488) (width 0.5) (layer F.Cu) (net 5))
 (segment (start 39.8 29.55) (end 39.8 22.64865) (width 0.5) (layer F.Cu) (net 5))
 (via (at 20.3 34.475) (size 0.8) (drill 0.4) (layers F.Cu B.Cu) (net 5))
 (segment (start 22.225 36.4) (end 20.3 34.475) (width 0.5) (layer B.Cu) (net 5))
 (segment (start 28.3 38.575) (end 26.125 36.4) (width 0.5) (layer B.Cu) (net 5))
 (segment (start 26.125 36.4) (end 22.225 36.4) (width 0.5) (layer B.Cu) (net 5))
 (segment (start 31.7779 34.9) (end 31.7779 37.0971) (width 0.5) (layer B.Cu) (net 5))
 (segment (start 31.7779 37.0971) (end 30.3 38.575) (width 0.5) (layer B.Cu) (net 5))
 (segment (start 34.3205 32.3574) (end 31.7779 34.9) (width 0.5) (layer B.Cu) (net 5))
 (segment (start 22.7414 40.6) (end 23.9 40.6) (width 0.5) (layer F.Cu) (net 4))
 (segment (start 23.9 41.875) (end 23.9 40.6) (width 0.5) (layer F.Cu) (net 4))
 (segment (start 21 40.525) (end 22.6664 40.525) (width 0.5) (layer B.Cu) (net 4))
 (segment (start 22.6664 40.525) (end 22.7414 40.6) (width 0.5) (layer B.Cu) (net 4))
 (via (at 22.7414 40.6) (size 0.8) (layers F.Cu B.Cu) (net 4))
 (segment (start 22.7414 40.6) (end 18.6478 36.5064) (width 0.5) (layer F.Cu) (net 4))
 (segment (start 18.6478 36.5064) (end 18.6478 27.4761) (width 0.5) (layer F.Cu) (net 4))
 (segment (start 18.6478 27.4761) (end 21.0239 25.1) (width 0.5) (layer F.Cu) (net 4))
 (segment (start 21.0239 20.9761) (end 24.3 17.7) (width 0.5) (layer F.Cu) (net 4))
 (segment (start 21.0239 25.1) (end 21.0239 20.9761) (width 0.5) (layer F.Cu) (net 4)))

